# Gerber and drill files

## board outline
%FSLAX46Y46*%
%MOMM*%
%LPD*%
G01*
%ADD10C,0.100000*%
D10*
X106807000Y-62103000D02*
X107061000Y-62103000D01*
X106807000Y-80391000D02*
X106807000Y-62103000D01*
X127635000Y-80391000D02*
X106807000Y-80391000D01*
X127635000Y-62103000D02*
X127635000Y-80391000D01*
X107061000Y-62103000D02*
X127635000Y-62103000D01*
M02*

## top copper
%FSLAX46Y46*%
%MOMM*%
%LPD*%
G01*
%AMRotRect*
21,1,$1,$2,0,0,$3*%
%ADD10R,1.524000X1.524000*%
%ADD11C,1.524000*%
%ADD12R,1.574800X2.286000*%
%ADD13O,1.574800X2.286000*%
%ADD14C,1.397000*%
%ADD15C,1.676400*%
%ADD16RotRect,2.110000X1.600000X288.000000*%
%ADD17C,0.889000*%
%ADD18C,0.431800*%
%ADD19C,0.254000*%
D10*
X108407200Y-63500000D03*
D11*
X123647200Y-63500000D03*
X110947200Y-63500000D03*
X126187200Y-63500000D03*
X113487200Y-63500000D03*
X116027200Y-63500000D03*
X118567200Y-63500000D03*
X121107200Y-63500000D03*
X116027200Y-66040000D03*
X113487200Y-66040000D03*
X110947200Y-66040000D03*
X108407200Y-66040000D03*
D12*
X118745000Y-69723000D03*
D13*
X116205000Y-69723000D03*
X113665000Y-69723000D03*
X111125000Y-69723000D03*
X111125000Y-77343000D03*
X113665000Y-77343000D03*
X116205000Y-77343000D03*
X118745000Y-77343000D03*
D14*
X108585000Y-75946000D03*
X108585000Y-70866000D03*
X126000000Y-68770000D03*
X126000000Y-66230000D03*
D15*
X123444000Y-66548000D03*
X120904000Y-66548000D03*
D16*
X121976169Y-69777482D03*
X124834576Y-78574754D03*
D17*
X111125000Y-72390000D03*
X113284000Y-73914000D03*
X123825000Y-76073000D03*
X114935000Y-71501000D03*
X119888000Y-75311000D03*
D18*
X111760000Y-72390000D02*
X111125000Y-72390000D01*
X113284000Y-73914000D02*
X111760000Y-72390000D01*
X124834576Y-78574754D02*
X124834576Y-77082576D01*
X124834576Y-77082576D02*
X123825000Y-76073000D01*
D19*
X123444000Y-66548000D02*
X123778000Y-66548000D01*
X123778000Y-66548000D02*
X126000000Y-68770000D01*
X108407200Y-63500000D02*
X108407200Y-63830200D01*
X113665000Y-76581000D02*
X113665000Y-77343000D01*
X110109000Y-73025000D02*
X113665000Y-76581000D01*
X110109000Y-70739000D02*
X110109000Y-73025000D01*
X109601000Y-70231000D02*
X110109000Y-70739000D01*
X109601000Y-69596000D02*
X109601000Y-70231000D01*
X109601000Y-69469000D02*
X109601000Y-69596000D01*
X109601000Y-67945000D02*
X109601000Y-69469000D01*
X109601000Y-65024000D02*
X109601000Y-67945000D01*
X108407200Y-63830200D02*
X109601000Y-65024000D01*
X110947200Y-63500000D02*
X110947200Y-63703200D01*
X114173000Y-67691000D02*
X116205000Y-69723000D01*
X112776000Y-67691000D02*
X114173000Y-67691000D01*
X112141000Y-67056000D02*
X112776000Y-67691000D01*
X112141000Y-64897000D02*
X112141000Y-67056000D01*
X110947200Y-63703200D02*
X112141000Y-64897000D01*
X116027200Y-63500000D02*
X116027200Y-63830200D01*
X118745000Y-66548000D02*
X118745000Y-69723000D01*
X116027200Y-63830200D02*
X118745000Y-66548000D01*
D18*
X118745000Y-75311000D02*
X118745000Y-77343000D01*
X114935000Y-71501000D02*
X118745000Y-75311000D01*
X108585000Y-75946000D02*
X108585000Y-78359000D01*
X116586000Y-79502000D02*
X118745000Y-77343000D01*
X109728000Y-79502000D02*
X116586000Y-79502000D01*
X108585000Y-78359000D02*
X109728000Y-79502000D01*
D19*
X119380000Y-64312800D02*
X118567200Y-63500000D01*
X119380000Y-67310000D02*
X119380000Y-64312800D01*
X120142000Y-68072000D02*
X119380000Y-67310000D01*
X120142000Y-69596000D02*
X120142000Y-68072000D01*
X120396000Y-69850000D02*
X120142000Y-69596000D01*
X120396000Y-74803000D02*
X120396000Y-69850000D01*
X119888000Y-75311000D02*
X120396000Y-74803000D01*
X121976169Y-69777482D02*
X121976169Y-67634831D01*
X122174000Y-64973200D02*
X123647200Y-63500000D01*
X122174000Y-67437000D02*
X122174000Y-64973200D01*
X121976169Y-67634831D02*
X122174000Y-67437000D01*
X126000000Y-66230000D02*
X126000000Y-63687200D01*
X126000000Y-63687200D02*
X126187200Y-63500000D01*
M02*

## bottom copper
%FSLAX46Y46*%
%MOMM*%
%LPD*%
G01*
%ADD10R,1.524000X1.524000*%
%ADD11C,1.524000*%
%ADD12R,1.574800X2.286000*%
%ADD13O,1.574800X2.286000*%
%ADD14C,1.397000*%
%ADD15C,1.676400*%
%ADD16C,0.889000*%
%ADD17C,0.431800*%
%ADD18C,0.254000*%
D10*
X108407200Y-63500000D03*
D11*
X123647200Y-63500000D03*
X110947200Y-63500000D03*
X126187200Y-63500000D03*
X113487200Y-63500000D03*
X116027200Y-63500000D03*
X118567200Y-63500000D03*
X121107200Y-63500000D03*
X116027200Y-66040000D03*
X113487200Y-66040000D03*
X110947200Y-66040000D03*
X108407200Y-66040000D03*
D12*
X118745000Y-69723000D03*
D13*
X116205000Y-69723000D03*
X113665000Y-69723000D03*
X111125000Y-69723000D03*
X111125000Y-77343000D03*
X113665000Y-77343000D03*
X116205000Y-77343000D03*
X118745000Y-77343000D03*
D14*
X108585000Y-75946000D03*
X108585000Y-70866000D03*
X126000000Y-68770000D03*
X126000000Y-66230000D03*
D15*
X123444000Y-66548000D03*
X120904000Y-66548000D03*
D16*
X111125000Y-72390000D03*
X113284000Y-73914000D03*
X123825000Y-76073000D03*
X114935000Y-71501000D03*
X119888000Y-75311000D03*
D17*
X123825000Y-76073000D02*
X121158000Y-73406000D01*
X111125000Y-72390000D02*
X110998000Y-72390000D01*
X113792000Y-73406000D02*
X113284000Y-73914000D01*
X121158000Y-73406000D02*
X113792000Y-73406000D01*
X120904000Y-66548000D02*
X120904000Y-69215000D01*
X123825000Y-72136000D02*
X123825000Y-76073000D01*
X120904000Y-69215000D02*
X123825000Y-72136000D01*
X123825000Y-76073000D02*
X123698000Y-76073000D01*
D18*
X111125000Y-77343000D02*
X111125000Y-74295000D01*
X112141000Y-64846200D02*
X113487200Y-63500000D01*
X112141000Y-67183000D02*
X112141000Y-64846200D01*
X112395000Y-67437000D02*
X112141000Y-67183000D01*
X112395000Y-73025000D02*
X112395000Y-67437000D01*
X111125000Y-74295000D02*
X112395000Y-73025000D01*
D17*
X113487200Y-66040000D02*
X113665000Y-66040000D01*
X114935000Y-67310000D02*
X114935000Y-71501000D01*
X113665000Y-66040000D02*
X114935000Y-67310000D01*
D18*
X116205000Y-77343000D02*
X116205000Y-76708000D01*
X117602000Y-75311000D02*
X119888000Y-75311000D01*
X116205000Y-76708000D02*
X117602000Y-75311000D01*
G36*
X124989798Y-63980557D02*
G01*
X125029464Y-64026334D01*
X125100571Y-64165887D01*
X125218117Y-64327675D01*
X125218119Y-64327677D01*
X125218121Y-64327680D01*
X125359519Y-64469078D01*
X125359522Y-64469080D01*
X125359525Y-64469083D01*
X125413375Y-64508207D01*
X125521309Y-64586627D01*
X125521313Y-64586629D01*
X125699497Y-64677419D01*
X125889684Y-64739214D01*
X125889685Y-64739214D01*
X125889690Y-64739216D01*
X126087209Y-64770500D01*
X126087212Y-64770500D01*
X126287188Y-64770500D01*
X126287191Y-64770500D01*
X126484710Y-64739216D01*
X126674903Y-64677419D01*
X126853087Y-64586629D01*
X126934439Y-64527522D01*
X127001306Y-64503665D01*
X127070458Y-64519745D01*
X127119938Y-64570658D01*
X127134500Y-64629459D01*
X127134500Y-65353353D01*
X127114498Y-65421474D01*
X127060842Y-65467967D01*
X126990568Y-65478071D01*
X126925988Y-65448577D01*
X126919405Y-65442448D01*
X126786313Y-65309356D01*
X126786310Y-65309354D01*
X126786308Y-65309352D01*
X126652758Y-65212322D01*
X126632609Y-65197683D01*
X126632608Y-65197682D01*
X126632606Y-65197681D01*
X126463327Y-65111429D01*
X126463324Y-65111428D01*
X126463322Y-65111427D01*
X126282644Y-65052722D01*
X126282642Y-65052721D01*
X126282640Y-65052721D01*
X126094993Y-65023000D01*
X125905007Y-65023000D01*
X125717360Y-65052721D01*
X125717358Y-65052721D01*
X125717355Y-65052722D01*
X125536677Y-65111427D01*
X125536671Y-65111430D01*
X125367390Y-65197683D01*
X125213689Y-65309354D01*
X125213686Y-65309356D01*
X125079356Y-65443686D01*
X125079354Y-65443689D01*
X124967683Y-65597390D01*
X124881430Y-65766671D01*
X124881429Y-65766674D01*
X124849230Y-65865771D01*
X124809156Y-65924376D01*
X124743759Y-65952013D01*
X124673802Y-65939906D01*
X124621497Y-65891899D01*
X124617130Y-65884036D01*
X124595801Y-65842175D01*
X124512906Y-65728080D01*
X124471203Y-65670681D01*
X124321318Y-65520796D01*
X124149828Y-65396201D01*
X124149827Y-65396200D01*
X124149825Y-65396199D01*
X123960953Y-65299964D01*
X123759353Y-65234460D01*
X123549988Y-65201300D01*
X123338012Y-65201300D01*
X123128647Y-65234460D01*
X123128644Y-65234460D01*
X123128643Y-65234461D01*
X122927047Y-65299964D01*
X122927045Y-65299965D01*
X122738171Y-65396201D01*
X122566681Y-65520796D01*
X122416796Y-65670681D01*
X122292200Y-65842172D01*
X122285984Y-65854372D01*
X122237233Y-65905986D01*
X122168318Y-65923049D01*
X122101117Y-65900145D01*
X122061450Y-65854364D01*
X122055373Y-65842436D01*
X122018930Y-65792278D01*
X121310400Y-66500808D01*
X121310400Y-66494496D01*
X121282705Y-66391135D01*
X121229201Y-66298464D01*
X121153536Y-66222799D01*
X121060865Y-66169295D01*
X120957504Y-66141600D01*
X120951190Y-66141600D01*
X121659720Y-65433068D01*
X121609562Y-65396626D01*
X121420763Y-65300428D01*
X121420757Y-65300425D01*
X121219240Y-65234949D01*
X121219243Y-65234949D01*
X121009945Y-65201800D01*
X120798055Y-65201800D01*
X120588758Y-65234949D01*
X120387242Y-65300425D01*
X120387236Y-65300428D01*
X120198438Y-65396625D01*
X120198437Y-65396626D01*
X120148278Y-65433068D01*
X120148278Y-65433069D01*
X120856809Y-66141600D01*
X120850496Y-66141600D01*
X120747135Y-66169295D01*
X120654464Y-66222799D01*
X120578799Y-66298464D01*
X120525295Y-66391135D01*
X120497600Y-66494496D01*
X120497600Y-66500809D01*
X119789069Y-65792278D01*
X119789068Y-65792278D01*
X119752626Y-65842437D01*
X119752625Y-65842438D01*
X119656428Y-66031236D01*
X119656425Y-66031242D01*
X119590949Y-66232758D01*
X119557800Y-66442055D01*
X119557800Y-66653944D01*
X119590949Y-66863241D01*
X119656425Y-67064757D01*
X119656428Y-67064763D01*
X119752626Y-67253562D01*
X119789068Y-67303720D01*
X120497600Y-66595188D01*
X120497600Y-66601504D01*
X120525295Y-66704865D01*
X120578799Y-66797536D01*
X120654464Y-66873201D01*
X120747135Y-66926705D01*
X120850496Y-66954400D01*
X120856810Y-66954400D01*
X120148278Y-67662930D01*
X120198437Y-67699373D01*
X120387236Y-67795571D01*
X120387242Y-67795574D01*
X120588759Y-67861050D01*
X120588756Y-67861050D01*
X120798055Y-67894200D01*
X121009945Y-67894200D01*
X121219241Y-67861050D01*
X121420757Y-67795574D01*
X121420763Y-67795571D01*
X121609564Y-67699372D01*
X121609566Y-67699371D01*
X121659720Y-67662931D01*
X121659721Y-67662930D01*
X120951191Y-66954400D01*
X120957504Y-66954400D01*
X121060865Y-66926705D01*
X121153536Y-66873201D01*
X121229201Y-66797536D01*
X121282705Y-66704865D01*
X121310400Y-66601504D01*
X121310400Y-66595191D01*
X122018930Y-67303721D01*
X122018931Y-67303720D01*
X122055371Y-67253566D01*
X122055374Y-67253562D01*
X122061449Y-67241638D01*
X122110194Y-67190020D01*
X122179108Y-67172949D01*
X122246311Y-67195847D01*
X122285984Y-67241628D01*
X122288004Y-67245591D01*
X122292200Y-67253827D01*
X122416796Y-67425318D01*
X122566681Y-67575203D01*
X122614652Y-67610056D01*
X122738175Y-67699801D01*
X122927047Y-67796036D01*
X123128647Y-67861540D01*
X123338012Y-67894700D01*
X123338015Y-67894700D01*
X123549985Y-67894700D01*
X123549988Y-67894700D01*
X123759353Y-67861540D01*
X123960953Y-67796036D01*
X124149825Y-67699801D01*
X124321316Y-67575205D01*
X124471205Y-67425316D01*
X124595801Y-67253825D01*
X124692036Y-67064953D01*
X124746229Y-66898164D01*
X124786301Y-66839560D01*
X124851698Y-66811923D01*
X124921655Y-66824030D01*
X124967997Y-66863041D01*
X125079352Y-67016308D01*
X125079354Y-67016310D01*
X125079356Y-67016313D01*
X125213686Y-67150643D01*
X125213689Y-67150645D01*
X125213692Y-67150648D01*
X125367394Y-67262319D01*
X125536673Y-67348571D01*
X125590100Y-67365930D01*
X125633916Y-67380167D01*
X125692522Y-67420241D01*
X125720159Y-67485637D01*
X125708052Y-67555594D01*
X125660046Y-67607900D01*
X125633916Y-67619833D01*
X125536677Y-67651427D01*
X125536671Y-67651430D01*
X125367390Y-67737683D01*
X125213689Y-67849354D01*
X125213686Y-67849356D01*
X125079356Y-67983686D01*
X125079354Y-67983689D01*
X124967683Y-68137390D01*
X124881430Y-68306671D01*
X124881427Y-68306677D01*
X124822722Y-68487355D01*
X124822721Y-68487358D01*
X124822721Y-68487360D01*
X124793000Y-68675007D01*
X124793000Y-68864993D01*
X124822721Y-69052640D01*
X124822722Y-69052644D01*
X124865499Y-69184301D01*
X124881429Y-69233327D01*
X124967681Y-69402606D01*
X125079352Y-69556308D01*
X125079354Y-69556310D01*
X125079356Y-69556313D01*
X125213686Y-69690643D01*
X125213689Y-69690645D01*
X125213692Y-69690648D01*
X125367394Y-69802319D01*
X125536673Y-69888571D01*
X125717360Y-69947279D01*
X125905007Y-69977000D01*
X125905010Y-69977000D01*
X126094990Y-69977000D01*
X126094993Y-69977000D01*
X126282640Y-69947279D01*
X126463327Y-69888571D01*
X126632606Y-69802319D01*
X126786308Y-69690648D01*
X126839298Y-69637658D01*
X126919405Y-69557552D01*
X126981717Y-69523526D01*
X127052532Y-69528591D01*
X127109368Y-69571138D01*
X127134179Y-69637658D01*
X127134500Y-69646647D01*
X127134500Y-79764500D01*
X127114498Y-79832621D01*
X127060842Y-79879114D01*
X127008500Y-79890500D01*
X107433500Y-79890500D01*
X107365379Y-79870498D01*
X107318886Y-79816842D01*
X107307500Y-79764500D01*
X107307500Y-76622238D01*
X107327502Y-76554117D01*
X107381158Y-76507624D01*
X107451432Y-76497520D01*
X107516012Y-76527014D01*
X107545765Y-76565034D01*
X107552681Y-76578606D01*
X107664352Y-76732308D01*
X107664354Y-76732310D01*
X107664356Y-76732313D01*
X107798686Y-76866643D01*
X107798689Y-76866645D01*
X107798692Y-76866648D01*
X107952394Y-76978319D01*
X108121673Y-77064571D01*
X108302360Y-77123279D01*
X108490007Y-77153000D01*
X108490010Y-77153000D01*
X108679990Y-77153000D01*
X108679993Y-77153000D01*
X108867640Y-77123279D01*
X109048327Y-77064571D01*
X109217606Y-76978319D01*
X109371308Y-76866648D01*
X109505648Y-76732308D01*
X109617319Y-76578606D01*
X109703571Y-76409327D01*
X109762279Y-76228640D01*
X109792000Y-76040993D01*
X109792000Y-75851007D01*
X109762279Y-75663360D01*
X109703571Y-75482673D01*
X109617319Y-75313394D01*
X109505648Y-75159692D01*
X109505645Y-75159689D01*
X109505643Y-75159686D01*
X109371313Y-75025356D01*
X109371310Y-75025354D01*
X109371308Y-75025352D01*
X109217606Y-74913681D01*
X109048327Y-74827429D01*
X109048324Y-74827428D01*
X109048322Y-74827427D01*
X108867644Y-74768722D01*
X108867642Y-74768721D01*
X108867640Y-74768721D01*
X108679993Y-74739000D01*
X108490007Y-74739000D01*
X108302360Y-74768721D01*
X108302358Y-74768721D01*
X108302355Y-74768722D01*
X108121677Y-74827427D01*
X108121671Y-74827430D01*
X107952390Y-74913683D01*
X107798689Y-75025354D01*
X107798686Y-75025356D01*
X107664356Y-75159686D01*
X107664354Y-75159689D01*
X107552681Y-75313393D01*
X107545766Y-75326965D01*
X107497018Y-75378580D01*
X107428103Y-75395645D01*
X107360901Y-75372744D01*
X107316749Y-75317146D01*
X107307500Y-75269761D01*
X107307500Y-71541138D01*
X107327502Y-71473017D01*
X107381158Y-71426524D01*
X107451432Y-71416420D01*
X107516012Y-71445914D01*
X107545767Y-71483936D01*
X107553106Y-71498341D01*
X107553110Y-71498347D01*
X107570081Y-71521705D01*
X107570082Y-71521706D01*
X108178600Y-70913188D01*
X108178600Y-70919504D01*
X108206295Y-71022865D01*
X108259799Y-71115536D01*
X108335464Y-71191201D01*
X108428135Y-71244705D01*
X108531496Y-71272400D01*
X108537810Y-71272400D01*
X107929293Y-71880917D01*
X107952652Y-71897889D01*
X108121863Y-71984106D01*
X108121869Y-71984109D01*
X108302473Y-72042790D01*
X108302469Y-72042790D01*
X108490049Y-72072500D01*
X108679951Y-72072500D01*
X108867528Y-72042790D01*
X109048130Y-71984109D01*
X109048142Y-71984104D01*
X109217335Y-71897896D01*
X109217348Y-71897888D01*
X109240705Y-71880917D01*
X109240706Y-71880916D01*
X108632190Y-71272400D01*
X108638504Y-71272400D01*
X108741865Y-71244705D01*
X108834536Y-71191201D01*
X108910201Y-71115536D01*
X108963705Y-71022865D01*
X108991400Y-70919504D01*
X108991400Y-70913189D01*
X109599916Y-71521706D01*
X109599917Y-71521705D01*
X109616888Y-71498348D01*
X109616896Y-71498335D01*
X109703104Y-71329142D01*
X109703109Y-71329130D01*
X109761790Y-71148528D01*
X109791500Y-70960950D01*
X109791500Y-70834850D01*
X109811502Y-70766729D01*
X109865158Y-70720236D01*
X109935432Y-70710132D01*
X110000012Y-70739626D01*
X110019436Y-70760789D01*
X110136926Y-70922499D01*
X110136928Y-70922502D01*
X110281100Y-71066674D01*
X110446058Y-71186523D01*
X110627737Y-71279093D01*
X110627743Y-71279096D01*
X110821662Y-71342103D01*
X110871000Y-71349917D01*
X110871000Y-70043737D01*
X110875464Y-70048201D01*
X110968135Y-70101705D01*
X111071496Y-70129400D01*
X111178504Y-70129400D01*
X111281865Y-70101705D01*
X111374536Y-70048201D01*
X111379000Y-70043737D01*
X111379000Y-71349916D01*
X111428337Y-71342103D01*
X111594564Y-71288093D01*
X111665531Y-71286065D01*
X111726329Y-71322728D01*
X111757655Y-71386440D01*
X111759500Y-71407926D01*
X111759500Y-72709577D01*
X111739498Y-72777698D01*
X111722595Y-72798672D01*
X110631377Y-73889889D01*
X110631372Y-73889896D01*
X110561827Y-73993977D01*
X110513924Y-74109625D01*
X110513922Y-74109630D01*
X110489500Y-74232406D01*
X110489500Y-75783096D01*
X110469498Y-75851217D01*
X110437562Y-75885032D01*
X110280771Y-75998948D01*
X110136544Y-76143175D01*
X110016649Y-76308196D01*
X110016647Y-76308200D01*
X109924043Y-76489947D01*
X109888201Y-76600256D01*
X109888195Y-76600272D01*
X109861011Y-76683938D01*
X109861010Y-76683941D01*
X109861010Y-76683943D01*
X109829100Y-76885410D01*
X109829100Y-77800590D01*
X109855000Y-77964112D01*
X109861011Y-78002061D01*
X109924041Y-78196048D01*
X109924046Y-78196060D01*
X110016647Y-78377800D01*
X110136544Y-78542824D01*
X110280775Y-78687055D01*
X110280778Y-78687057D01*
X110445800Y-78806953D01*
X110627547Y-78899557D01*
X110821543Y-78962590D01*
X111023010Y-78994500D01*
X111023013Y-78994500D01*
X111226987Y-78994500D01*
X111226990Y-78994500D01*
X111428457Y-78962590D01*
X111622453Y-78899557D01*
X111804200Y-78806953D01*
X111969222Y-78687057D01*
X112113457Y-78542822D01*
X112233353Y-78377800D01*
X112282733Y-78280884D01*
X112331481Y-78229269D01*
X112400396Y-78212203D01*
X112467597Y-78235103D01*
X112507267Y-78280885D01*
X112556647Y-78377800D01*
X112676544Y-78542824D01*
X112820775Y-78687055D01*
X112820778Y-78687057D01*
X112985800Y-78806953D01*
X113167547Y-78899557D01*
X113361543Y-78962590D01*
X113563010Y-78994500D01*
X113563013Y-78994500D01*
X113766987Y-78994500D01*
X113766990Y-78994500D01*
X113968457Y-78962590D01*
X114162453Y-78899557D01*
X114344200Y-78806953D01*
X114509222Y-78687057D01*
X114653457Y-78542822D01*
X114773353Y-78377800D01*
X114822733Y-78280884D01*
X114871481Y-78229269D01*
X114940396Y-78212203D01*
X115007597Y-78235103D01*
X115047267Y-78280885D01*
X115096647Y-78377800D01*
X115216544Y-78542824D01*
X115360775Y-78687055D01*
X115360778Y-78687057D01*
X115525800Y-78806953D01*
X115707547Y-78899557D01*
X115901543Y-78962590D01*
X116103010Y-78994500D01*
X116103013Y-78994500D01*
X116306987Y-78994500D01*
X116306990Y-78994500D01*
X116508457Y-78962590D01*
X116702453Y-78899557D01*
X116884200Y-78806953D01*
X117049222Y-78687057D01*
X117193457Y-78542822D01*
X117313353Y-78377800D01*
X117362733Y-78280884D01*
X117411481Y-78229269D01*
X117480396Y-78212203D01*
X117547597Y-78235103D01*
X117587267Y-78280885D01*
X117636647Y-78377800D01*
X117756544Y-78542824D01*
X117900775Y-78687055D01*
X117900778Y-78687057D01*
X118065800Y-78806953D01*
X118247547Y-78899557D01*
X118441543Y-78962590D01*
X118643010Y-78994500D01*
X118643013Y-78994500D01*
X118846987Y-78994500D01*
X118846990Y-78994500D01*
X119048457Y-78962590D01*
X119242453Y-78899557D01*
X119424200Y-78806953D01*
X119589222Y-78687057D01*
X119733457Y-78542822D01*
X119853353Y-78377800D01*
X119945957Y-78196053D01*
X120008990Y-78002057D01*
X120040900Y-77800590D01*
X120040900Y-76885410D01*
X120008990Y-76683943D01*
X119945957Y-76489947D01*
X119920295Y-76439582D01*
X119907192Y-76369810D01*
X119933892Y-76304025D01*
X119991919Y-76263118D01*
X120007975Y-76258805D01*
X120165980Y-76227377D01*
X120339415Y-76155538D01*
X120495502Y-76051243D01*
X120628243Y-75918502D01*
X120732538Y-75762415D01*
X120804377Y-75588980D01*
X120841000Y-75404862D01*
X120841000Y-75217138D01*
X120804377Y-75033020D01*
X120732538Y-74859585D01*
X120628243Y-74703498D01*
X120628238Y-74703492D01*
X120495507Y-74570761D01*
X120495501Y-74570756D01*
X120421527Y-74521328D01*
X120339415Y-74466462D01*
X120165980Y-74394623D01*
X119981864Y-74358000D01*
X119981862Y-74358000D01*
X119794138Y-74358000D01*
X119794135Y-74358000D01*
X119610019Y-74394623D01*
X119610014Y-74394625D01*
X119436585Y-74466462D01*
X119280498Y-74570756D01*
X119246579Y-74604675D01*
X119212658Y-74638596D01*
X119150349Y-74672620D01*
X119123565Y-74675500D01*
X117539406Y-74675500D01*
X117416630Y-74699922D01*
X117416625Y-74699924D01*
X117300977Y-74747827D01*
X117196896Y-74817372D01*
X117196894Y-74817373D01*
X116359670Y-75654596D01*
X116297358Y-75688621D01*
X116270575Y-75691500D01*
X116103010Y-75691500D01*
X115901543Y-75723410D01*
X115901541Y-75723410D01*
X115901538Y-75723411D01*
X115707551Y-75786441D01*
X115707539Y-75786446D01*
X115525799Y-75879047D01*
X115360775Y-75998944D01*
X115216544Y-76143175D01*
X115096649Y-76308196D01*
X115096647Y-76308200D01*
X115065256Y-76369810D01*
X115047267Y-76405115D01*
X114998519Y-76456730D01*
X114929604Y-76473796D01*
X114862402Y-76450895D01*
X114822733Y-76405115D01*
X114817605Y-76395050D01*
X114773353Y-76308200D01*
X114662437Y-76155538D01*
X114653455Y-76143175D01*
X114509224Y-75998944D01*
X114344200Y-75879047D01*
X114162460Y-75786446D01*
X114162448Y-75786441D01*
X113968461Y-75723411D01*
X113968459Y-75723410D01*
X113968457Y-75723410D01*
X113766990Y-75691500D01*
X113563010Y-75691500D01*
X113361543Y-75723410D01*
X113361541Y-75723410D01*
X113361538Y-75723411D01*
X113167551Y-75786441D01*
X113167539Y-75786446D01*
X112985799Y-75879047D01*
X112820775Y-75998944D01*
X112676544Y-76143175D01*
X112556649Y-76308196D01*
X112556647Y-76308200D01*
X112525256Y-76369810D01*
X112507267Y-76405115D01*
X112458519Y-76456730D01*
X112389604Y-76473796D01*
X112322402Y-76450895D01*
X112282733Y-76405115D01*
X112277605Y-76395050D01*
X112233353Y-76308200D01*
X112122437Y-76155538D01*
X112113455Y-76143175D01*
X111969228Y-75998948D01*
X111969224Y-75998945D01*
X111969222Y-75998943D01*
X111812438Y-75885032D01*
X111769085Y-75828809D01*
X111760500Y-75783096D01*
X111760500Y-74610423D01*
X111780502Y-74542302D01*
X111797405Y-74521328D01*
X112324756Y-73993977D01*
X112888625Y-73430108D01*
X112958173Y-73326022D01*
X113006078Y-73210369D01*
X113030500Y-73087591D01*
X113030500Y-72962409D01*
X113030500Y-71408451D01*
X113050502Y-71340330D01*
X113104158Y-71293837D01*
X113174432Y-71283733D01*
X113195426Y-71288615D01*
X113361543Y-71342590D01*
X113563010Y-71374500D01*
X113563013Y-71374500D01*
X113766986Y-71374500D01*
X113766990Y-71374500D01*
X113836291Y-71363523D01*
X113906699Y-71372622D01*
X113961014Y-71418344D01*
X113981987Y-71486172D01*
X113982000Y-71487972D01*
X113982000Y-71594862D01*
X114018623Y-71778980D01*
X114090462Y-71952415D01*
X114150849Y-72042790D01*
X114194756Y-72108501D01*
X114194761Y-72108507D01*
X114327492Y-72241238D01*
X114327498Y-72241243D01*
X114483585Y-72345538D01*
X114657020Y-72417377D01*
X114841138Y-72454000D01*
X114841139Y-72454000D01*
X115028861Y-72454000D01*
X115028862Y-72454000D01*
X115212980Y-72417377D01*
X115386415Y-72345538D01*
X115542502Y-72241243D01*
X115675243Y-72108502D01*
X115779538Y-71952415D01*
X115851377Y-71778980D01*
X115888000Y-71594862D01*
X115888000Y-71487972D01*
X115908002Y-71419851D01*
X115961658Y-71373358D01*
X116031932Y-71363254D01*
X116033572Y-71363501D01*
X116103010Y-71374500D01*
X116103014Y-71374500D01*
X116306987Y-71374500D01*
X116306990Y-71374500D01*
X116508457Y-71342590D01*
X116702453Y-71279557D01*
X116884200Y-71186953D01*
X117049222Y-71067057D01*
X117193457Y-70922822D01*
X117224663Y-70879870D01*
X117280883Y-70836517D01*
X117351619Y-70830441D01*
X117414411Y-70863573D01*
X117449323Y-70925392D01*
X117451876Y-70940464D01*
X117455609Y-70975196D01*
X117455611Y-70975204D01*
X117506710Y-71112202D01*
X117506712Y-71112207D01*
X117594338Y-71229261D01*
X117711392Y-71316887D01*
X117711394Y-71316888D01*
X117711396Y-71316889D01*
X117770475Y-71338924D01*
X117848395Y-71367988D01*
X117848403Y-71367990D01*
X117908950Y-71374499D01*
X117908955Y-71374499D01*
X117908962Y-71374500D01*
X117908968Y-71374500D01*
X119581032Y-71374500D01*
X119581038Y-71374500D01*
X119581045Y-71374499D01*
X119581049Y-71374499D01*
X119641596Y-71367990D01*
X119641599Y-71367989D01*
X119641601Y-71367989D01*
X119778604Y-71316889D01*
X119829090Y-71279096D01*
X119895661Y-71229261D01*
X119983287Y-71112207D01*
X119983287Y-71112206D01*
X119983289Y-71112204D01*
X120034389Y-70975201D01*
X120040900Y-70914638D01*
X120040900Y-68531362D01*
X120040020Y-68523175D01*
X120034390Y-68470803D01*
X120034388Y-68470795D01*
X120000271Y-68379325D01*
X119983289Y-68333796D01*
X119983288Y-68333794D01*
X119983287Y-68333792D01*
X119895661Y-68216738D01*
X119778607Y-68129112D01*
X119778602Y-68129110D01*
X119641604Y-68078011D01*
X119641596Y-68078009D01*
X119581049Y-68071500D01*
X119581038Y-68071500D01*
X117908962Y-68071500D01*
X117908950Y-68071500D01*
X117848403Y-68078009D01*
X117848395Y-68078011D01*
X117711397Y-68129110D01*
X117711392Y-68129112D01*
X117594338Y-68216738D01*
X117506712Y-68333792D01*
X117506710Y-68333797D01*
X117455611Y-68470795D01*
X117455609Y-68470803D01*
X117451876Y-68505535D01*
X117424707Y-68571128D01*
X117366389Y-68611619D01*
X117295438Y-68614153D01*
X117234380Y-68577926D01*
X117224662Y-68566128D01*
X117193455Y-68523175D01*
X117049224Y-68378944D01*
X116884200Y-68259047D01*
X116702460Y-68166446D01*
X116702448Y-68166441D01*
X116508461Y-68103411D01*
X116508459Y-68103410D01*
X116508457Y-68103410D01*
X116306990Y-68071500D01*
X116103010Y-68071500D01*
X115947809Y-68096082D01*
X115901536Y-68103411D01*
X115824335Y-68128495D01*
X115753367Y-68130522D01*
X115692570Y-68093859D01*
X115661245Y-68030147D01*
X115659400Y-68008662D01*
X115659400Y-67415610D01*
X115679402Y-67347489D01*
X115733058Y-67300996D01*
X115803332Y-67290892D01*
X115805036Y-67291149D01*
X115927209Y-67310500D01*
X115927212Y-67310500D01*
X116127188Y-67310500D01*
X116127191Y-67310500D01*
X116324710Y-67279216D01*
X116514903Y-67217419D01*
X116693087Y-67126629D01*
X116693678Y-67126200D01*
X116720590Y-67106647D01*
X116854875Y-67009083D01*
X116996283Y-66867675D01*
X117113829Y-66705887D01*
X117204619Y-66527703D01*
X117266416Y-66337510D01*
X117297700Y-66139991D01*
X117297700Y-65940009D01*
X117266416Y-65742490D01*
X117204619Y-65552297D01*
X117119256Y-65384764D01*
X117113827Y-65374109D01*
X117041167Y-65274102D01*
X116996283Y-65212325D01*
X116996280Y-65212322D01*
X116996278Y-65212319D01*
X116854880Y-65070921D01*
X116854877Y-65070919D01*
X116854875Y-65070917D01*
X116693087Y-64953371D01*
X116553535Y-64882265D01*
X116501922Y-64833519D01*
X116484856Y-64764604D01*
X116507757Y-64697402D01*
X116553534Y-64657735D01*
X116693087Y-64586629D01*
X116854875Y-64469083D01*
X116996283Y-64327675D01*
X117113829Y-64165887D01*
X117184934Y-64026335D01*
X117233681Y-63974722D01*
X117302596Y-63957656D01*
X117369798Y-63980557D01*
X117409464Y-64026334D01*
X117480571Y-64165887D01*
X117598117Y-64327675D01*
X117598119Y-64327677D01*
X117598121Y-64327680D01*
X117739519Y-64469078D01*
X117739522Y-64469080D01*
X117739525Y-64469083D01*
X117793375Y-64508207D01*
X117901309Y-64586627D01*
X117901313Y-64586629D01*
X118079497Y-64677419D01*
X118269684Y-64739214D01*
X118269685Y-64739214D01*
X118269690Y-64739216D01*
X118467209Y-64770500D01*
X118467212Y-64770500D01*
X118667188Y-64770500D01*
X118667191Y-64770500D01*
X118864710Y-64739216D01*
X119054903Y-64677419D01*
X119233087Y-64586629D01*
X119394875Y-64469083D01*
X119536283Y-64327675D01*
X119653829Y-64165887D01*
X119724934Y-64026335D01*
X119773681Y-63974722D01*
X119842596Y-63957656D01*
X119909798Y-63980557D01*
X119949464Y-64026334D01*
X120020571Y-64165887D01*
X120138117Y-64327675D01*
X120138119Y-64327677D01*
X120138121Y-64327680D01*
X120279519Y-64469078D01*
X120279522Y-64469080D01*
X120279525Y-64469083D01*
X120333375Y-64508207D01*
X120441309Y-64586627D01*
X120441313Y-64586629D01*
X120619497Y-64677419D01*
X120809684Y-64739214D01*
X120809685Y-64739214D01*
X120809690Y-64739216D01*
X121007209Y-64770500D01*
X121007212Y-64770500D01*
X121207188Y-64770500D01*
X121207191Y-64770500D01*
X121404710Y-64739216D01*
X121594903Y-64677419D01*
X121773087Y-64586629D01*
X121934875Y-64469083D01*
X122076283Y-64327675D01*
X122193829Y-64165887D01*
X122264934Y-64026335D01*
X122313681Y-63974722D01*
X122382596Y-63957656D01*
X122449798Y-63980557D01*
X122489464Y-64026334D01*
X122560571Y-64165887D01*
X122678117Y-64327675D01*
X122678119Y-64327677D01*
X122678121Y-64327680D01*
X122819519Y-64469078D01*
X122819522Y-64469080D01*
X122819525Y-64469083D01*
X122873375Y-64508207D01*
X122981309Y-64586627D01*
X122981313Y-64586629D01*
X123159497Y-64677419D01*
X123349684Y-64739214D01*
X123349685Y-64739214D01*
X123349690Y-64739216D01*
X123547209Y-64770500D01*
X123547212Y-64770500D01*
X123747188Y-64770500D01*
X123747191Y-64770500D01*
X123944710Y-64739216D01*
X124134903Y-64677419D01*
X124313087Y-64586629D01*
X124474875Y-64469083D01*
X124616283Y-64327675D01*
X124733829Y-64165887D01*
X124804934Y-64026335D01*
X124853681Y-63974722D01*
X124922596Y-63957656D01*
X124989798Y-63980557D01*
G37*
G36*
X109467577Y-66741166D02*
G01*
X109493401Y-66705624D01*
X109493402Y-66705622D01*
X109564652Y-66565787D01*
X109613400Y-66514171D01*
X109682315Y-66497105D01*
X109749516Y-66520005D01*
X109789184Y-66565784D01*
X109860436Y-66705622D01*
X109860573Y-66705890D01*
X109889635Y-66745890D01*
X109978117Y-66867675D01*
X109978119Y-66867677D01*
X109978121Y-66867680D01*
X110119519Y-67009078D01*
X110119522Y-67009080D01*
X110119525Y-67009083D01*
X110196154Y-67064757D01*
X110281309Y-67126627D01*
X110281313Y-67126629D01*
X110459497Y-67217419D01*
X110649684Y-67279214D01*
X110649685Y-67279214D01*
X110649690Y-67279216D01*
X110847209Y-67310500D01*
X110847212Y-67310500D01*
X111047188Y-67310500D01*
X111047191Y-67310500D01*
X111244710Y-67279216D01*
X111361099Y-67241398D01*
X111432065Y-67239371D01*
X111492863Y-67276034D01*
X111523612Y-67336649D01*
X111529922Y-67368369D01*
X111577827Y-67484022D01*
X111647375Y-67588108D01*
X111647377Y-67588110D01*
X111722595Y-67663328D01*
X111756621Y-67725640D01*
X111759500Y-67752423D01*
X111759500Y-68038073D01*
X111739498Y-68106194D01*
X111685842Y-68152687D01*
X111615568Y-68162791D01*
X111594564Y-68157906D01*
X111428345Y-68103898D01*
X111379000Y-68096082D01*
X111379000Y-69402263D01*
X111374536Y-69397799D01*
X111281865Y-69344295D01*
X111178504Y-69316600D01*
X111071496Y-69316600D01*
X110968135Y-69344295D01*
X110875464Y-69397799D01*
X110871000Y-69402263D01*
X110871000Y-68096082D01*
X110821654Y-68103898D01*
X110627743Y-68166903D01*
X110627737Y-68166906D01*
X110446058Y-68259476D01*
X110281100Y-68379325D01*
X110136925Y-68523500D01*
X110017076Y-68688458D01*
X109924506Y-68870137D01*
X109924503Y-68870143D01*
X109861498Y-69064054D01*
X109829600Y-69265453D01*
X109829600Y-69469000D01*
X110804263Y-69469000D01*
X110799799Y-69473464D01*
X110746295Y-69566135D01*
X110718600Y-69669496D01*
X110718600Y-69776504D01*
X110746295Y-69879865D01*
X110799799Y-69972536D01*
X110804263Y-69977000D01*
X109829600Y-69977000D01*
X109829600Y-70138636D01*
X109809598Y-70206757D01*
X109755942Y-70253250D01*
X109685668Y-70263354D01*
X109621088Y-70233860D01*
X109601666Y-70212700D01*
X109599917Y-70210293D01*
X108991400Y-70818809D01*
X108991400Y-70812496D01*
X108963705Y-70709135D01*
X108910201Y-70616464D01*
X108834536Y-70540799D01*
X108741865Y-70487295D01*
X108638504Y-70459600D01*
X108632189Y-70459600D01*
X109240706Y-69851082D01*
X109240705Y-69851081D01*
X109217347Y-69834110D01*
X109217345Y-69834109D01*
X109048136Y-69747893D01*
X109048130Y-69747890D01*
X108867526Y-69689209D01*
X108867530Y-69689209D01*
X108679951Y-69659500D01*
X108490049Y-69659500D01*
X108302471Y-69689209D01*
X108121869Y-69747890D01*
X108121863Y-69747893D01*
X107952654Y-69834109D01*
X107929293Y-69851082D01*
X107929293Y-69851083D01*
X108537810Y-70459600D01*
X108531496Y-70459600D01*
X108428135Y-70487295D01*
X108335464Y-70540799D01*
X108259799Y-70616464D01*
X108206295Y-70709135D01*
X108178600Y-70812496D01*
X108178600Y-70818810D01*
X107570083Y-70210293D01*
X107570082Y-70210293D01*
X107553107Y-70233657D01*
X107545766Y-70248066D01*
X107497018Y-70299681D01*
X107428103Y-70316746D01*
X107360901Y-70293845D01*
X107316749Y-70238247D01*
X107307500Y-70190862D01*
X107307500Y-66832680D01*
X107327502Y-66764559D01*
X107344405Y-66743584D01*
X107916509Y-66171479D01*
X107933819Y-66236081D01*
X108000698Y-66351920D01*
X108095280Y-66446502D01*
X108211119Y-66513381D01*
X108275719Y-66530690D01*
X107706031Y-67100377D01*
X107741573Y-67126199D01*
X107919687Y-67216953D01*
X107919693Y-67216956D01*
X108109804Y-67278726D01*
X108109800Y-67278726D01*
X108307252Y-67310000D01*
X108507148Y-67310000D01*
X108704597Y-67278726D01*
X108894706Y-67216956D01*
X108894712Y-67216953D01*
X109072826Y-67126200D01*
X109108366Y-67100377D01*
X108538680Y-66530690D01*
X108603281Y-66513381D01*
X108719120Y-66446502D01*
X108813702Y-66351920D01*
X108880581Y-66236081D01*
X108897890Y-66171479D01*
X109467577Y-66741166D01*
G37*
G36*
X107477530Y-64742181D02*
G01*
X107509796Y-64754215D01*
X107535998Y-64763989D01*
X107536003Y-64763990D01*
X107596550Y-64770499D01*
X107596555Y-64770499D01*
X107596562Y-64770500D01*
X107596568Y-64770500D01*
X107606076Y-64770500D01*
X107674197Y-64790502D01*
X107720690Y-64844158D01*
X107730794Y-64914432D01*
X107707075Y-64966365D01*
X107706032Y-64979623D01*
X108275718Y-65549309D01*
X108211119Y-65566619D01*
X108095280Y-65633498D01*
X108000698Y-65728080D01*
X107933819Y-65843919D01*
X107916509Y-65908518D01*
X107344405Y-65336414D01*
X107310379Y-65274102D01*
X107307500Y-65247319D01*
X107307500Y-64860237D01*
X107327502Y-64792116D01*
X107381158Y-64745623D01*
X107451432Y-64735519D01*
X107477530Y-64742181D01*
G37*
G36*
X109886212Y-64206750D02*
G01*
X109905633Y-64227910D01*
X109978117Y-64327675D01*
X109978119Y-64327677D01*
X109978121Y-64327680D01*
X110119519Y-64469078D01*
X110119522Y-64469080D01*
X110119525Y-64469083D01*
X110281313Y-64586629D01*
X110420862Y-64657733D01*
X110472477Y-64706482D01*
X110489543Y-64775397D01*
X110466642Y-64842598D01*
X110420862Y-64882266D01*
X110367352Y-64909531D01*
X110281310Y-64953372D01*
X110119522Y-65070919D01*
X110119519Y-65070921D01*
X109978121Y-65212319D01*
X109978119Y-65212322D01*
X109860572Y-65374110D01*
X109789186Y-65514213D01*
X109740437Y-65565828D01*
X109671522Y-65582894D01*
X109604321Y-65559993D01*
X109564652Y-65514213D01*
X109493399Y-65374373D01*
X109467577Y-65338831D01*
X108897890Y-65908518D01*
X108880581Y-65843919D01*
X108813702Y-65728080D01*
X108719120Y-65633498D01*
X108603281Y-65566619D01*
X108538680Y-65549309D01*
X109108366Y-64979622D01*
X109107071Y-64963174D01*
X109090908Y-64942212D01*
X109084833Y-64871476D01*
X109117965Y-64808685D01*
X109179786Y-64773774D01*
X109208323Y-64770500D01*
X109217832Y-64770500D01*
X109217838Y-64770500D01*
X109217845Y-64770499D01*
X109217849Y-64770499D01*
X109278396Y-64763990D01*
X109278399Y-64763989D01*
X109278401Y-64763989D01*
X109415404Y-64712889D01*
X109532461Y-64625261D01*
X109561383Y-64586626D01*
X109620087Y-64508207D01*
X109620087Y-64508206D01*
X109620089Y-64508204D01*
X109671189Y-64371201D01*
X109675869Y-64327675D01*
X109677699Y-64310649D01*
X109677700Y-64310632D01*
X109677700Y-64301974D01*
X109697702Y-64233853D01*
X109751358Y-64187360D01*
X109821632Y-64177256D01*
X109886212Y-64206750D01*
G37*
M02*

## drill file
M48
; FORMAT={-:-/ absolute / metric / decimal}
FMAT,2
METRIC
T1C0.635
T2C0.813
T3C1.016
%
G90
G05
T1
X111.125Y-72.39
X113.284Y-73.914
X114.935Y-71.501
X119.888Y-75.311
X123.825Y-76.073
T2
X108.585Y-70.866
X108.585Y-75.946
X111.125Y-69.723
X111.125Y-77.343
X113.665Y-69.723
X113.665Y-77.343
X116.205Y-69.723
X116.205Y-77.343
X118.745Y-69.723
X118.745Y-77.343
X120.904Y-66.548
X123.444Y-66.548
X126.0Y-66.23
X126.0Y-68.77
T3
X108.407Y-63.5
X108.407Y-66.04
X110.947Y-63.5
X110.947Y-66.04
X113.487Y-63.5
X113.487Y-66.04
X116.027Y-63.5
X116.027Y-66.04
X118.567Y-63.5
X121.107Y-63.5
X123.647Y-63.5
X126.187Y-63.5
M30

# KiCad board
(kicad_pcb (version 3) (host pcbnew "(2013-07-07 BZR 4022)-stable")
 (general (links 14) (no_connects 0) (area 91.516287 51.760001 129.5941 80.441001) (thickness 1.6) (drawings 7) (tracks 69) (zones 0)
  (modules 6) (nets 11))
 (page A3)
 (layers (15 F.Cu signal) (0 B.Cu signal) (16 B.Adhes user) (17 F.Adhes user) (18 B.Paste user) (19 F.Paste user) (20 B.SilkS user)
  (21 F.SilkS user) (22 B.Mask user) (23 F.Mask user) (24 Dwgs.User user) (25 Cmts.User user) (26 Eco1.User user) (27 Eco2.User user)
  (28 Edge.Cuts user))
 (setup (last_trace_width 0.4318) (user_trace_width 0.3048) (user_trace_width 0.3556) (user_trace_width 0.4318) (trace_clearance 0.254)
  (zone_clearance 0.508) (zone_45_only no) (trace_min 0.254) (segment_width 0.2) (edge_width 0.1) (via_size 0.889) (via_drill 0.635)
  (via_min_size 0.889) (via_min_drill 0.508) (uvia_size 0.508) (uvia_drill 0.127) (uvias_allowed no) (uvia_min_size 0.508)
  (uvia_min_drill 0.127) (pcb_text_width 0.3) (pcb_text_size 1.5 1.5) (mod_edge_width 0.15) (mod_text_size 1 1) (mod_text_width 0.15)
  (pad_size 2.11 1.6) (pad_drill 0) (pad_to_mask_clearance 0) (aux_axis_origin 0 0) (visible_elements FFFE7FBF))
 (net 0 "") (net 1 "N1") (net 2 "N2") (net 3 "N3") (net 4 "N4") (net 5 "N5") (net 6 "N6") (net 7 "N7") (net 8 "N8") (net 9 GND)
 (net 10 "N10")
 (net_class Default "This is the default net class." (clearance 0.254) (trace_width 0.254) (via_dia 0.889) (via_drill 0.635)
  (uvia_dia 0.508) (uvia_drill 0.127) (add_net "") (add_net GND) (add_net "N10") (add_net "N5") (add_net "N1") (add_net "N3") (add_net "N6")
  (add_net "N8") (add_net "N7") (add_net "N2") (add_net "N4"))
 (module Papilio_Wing (layer F.Cu) (at 108.4072 63.5)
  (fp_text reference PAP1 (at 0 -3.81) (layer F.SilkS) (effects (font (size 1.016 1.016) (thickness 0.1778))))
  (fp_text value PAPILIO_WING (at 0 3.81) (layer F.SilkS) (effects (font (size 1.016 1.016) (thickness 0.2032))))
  (pad 1 thru_hole rect (at 0 0) (size 1.524 1.524) (drill 1.016) (layers *.Cu *.Mask F.SilkS) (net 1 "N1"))
  (pad 7 thru_hole circle (at 15.24 0) (size 1.524 1.524) (drill 1.016) (layers *.Cu *.Mask F.SilkS) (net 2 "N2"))
  (pad 2 thru_hole circle (at 2.54 0) (size 1.524 1.524) (drill 1.016) (layers *.Cu *.Mask F.SilkS) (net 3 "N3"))
  (pad 8 thru_hole circle (at 17.78 0) (size 1.524 1.524) (drill 1.016) (layers *.Cu *.Mask F.SilkS) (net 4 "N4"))
  (pad 3 thru_hole circle (at 5.08 0) (size 1.524 1.524) (drill 1.016) (layers *.Cu *.Mask F.SilkS) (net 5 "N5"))
  (pad 4 thru_hole circle (at 7.62 0) (size 1.524 1.524) (drill 1.016) (layers *.Cu *.Mask F.SilkS) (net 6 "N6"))
  (pad 5 thru_hole circle (at 10.16 0) (size 1.524 1.524) (drill 1.016) (layers *.Cu *.Mask F.SilkS) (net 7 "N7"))
  (pad 6 thru_hole circle (at 12.7 0) (size 1.524 1.524) (drill 1.016) (layers *.Cu *.Mask F.SilkS))
  (pad 9 thru_hole circle (at 7.62 2.54) (size 1.524 1.524) (drill 1.016) (layers *.Cu *.Mask F.SilkS))
  (pad 10 thru_hole circle (at 5.08 2.54) (size 1.524 1.524) (drill 1.016) (layers *.Cu *.Mask F.SilkS) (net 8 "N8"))
  (pad 11 thru_hole circle (at 2.54 2.54) (size 1.524 1.524) (drill 1.016) (layers *.Cu *.Mask F.SilkS))
  (pad 12 thru_hole circle (at 0 2.54) (size 1.524 1.524) (drill 1.016) (layers *.Cu *.Mask F.SilkS) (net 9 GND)))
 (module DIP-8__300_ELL (layer F.Cu) (at 114.935 73.533 180)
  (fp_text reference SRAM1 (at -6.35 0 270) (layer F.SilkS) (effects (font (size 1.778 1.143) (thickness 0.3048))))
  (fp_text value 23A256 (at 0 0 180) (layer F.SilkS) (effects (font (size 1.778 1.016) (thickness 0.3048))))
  (pad 1 thru_hole rect (at -3.81 3.81 180) (size 1.5748 2.286) (drill 0.8128) (layers *.Cu *.Mask F.SilkS) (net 6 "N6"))
  (pad 2 thru_hole oval (at -1.27 3.81 180) (size 1.5748 2.286) (drill 0.8128) (layers *.Cu *.Mask F.SilkS) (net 3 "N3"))
  (pad 3 thru_hole oval (at 1.27 3.81 180) (size 1.5748 2.286) (drill 0.8128) (layers *.Cu *.Mask F.SilkS))
  (pad 4 thru_hole oval (at 3.81 3.81 180) (size 1.5748 2.286) (drill 0.8128) (layers *.Cu *.Mask F.SilkS) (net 9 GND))
  (pad 5 thru_hole oval (at 3.81 -3.81 180) (size 1.5748 2.286) (drill 0.8128) (layers *.Cu *.Mask F.SilkS) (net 5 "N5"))
  (pad 6 thru_hole oval (at 1.27 -3.81 180) (size 1.5748 2.286) (drill 0.8128) (layers *.Cu *.Mask F.SilkS) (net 1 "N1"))
  (pad 7 thru_hole oval (at -1.27 -3.81 180) (size 1.5748 2.286) (drill 0.8128) (layers *.Cu *.Mask F.SilkS) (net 7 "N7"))
  (pad 8 thru_hole oval (at -3.81 -3.81 180) (size 1.5748 2.286) (drill 0.8128) (layers *.Cu *.Mask F.SilkS) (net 8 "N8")))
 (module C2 (layer F.Cu) (at 108.585 73.406 90)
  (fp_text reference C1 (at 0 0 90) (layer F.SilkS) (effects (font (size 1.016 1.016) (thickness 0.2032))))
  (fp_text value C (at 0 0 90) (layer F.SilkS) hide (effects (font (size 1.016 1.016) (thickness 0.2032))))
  (pad 1 thru_hole circle (at -2.54 0 90) (size 1.397 1.397) (drill 0.8128) (layers *.Cu *.Mask F.SilkS) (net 8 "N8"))
  (pad 2 thru_hole circle (at 2.54 0 90) (size 1.397 1.397) (drill 0.8128) (layers *.Cu *.Mask F.SilkS) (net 9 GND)))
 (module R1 (layer F.Cu) (at 126 67.5 90) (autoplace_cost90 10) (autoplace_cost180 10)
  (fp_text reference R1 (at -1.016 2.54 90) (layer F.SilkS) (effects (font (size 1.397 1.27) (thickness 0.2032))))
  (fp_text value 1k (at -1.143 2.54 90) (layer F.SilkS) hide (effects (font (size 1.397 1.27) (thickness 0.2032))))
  (pad 1 thru_hole circle (at -1.27 0 90) (size 1.397 1.397) (drill 0.8128) (layers *.Cu *.Mask F.SilkS) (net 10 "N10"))
  (pad 2 thru_hole circle (at 1.27 0 90) (size 1.397 1.397) (drill 0.8128) (layers *.Cu *.Mask F.SilkS) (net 4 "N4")))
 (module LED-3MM (layer F.Cu) (at 122.174 66.548 180)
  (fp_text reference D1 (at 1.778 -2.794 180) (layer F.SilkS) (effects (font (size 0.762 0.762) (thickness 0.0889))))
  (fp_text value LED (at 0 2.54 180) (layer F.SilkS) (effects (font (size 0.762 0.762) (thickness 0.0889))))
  (pad 1 thru_hole circle (at -1.27 0 180) (size 1.6764 1.6764) (drill 0.8128) (layers *.Cu *.Mask F.SilkS) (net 10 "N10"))
  (pad 2 thru_hole circle (at 1.27 0 180) (size 1.6764 1.6764) (drill 0.8128) (layers *.Cu *.Mask F.SilkS) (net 9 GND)))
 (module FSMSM (layer F.Cu) (at 123.444 74.295 288)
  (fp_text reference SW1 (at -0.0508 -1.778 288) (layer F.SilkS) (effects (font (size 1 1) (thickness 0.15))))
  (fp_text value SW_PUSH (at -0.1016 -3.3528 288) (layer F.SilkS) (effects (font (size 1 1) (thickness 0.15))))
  (pad 1 smd rect (at -4.75 0 288) (size 2.11 1.6) (layers F.Cu F.Paste F.Mask) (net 2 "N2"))
  (pad 2 smd rect (at 4.5 0 288) (size 2.11 1.6) (layers F.Cu F.Paste F.Mask) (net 9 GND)))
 (gr_line (start 106.807 62.103) (end 107.061 62.103) (angle 90) (layer Edge.Cuts) (width 0.1))
 (gr_line (start 106.807 80.391) (end 106.807 62.103) (angle 90) (layer Edge.Cuts) (width 0.1))
 (gr_line (start 127.635 80.391) (end 106.807 80.391) (angle 90) (layer Edge.Cuts) (width 0.1))
 (gr_line (start 127.635 62.103) (end 127.635 80.391) (angle 90) (layer Edge.Cuts) (width 0.1))
 (gr_line (start 107.061 62.103) (end 127.635 62.103) (angle 90) (layer Edge.Cuts) (width 0.1))
 (segment (start 123.825 76.073) (end 121.158 73.406) (width 0.4318) (layer B.Cu) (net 9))
 (segment (start 111.125 72.39) (end 110.998 72.39) (width 0.4318) (layer B.Cu) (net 9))
 (via (at 111.125 72.39) (size 0.889) (layers F.Cu B.Cu) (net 9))
 (segment (start 111.76 72.39) (end 111.125 72.39) (width 0.4318) (layer F.Cu) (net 9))
 (segment (start 113.284 73.914) (end 111.76 72.39) (width 0.4318) (layer F.Cu) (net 9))
 (via (at 113.284 73.914) (size 0.889) (layers F.Cu B.Cu) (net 9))
 (segment (start 113.792 73.406) (end 113.284 73.914) (width 0.4318) (layer B.Cu) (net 9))
 (segment (start 121.158 73.406) (end 113.792 73.406) (width 0.4318) (layer B.Cu) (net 9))
 (segment (start 120.904 66.548) (end 120.904 69.215) (width 0.4318) (layer B.Cu) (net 9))
 (segment (start 123.825 72.136) (end 123.825 76.073) (width 0.4318) (layer B.Cu) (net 9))
 (segment (start 120.904 69.215) (end 123.825 72.136) (width 0.4318) (layer B.Cu) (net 9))
 (segment (start 124.834576 78.574754) (end 124.834576 77.082576) (width 0.4318) (layer F.Cu) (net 9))
 (segment (start 123.825 76.073) (end 123.698 76.073) (width 0.4318) (layer B.Cu) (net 9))
 (via (at 123.825 76.073) (size 0.889) (layers F.Cu B.Cu) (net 9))
 (segment (start 124.834576 77.082576) (end 123.825 76.073) (width 0.4318) (layer F.Cu) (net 9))
 (segment (start 123.444 66.548) (end 123.778 66.548) (width 0.254) (layer F.Cu) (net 10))
 (segment (start 123.778 66.548) (end 126 68.77) (width 0.254) (layer F.Cu) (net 10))
 (segment (start 111.125 77.343) (end 111.125 74.295) (width 0.254) (layer B.Cu) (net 5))
 (segment (start 112.141 64.8462) (end 113.4872 63.5) (width 0.254) (layer B.Cu) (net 5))
 (segment (start 112.141 67.183) (end 112.141 64.8462) (width 0.254) (layer B.Cu) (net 5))
 (segment (start 112.395 67.437) (end 112.141 67.183) (width 0.254) (layer B.Cu) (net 5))
 (segment (start 112.395 73.025) (end 112.395 67.437) (width 0.254) (layer B.Cu) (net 5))
 (segment (start 111.125 74.295) (end 112.395 73.025) (width 0.254) (layer B.Cu) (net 5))
 (segment (start 108.4072 63.5) (end 108.4072 63.8302) (width 0.254) (layer F.Cu) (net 1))
 (segment (start 113.665 76.581) (end 113.665 77.343) (width 0.254) (layer F.Cu) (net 1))
 (segment (start 110.109 73.025) (end 113.665 76.581) (width 0.254) (layer F.Cu) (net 1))
 (segment (start 110.109 70.739) (end 110.109 73.025) (width 0.254) (layer F.Cu) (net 1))
 (segment (start 109.601 70.231) (end 110.109 70.739) (width 0.254) (layer F.Cu) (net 1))
 (segment (start 109.601 69.596) (end 109.601 70.231) (width 0.254) (layer F.Cu) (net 1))
 (segment (start 109.601 69.469) (end 109.601 69.596) (width 0.254) (layer F.Cu) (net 1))
 (segment (start 109.601 67.945) (end 109.601 69.469) (width 0.254) (layer F.Cu) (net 1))
 (segment (start 109.601 65.024) (end 109.601 67.945) (width 0.254) (layer F.Cu) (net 1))
 (segment (start 108.4072 63.8302) (end 109.601 65.024) (width 0.254) (layer F.Cu) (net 1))
 (segment (start 110.9472 63.5) (end 110.9472 63.7032) (width 0.254) (layer F.Cu) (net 3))
 (segment (start 114.173 67.691) (end 116.205 69.723) (width 0.254) (layer F.Cu) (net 3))
 (segment (start 112.776 67.691) (end 114.173 67.691) (width 0.254) (layer F.Cu) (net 3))
 (segment (start 112.141 67.056) (end 112.776 67.691) (width 0.254) (layer F.Cu) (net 3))
 (segment (start 112.141 64.897) (end 112.141 67.056) (width 0.254) (layer F.Cu) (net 3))
 (segment (start 110.9472 63.7032) (end 112.141 64.897) (width 0.254) (layer F.Cu) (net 3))
 (segment (start 116.0272 63.5) (end 116.0272 63.8302) (width 0.254) (layer F.Cu) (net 6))
 (segment (start 118.745 66.548) (end 118.745 69.723) (width 0.254) (layer F.Cu) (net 6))
 (segment (start 116.0272 63.8302) (end 118.745 66.548) (width 0.254) (layer F.Cu) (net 6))
 (segment (start 113.4872 66.04) (end 113.665 66.04) (width 0.4318) (layer B.Cu) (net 8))
 (segment (start 118.745 75.311) (end 118.745 77.343) (width 0.4318) (layer F.Cu) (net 8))
 (segment (start 114.935 71.501) (end 118.745 75.311) (width 0.4318) (layer F.Cu) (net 8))
 (via (at 114.935 71.501) (size 0.889) (layers F.Cu B.Cu) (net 8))
 (segment (start 114.935 67.31) (end 114.935 71.501) (width 0.4318) (layer B.Cu) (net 8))
 (segment (start 113.665 66.04) (end 114.935 67.31) (width 0.4318) (layer B.Cu) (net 8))
 (segment (start 108.585 75.946) (end 108.585 78.359) (width 0.4318) (layer F.Cu) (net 8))
 (segment (start 116.586 79.502) (end 118.745 77.343) (width 0.4318) (layer F.Cu) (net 8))
 (segment (start 109.728 79.502) (end 116.586 79.502) (width 0.4318) (layer F.Cu) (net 8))
 (segment (start 108.585 78.359) (end 109.728 79.502) (width 0.4318) (layer F.Cu) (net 8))
 (segment (start 116.205 77.343) (end 116.205 76.708) (width 0.254) (layer B.Cu) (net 7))
 (segment (start 119.38 64.3128) (end 118.5672 63.5) (width 0.254) (layer F.Cu) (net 7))
 (segment (start 119.38 67.31) (end 119.38 64.3128) (width 0.254) (layer F.Cu) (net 7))
 (segment (start 120.142 68.072) (end 119.38 67.31) (width 0.254) (layer F.Cu) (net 7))
 (segment (start 120.142 69.596) (end 120.142 68.072) (width 0.254) (layer F.Cu) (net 7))
 (segment (start 120.396 69.85) (end 120.142 69.596) (width 0.254) (layer F.Cu) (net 7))
 (segment (start 120.396 74.803) (end 120.396 69.85) (width 0.254) (layer F.Cu) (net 7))
 (segment (start 119.888 75.311) (end 120.396 74.803) (width 0.254) (layer F.Cu) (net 7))
 (via (at 119.888 75.311) (size 0.889) (layers F.Cu B.Cu) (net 7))
 (segment (start 117.602 75.311) (end 119.888 75.311) (width 0.254) (layer B.Cu) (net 7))
 (segment (start 116.205 76.708) (end 117.602 75.311) (width 0.254) (layer B.Cu) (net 7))
 (segment (start 121.976169 69.777482) (end 121.976169 67.634831) (width 0.254) (layer F.Cu) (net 2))
 (segment (start 122.174 64.9732) (end 123.6472 63.5) (width 0.254) (layer F.Cu) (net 2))
 (segment (start 122.174 67.437) (end 122.174 64.9732) (width 0.254) (layer F.Cu) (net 2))
 (segment (start 121.976169 67.634831) (end 122.174 67.437) (width 0.254) (layer F.Cu) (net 2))
 (segment (start 126 66.23) (end 126 63.6872) (width 0.254) (layer F.Cu) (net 4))
 (segment (start 126 63.6872) (end 126.1872 63.5) (width 0.254) (layer F.Cu) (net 4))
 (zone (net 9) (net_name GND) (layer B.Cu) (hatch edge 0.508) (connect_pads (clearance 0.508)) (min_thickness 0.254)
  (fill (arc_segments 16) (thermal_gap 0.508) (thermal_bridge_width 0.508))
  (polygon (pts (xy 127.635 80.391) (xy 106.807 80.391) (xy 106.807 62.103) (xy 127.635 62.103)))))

